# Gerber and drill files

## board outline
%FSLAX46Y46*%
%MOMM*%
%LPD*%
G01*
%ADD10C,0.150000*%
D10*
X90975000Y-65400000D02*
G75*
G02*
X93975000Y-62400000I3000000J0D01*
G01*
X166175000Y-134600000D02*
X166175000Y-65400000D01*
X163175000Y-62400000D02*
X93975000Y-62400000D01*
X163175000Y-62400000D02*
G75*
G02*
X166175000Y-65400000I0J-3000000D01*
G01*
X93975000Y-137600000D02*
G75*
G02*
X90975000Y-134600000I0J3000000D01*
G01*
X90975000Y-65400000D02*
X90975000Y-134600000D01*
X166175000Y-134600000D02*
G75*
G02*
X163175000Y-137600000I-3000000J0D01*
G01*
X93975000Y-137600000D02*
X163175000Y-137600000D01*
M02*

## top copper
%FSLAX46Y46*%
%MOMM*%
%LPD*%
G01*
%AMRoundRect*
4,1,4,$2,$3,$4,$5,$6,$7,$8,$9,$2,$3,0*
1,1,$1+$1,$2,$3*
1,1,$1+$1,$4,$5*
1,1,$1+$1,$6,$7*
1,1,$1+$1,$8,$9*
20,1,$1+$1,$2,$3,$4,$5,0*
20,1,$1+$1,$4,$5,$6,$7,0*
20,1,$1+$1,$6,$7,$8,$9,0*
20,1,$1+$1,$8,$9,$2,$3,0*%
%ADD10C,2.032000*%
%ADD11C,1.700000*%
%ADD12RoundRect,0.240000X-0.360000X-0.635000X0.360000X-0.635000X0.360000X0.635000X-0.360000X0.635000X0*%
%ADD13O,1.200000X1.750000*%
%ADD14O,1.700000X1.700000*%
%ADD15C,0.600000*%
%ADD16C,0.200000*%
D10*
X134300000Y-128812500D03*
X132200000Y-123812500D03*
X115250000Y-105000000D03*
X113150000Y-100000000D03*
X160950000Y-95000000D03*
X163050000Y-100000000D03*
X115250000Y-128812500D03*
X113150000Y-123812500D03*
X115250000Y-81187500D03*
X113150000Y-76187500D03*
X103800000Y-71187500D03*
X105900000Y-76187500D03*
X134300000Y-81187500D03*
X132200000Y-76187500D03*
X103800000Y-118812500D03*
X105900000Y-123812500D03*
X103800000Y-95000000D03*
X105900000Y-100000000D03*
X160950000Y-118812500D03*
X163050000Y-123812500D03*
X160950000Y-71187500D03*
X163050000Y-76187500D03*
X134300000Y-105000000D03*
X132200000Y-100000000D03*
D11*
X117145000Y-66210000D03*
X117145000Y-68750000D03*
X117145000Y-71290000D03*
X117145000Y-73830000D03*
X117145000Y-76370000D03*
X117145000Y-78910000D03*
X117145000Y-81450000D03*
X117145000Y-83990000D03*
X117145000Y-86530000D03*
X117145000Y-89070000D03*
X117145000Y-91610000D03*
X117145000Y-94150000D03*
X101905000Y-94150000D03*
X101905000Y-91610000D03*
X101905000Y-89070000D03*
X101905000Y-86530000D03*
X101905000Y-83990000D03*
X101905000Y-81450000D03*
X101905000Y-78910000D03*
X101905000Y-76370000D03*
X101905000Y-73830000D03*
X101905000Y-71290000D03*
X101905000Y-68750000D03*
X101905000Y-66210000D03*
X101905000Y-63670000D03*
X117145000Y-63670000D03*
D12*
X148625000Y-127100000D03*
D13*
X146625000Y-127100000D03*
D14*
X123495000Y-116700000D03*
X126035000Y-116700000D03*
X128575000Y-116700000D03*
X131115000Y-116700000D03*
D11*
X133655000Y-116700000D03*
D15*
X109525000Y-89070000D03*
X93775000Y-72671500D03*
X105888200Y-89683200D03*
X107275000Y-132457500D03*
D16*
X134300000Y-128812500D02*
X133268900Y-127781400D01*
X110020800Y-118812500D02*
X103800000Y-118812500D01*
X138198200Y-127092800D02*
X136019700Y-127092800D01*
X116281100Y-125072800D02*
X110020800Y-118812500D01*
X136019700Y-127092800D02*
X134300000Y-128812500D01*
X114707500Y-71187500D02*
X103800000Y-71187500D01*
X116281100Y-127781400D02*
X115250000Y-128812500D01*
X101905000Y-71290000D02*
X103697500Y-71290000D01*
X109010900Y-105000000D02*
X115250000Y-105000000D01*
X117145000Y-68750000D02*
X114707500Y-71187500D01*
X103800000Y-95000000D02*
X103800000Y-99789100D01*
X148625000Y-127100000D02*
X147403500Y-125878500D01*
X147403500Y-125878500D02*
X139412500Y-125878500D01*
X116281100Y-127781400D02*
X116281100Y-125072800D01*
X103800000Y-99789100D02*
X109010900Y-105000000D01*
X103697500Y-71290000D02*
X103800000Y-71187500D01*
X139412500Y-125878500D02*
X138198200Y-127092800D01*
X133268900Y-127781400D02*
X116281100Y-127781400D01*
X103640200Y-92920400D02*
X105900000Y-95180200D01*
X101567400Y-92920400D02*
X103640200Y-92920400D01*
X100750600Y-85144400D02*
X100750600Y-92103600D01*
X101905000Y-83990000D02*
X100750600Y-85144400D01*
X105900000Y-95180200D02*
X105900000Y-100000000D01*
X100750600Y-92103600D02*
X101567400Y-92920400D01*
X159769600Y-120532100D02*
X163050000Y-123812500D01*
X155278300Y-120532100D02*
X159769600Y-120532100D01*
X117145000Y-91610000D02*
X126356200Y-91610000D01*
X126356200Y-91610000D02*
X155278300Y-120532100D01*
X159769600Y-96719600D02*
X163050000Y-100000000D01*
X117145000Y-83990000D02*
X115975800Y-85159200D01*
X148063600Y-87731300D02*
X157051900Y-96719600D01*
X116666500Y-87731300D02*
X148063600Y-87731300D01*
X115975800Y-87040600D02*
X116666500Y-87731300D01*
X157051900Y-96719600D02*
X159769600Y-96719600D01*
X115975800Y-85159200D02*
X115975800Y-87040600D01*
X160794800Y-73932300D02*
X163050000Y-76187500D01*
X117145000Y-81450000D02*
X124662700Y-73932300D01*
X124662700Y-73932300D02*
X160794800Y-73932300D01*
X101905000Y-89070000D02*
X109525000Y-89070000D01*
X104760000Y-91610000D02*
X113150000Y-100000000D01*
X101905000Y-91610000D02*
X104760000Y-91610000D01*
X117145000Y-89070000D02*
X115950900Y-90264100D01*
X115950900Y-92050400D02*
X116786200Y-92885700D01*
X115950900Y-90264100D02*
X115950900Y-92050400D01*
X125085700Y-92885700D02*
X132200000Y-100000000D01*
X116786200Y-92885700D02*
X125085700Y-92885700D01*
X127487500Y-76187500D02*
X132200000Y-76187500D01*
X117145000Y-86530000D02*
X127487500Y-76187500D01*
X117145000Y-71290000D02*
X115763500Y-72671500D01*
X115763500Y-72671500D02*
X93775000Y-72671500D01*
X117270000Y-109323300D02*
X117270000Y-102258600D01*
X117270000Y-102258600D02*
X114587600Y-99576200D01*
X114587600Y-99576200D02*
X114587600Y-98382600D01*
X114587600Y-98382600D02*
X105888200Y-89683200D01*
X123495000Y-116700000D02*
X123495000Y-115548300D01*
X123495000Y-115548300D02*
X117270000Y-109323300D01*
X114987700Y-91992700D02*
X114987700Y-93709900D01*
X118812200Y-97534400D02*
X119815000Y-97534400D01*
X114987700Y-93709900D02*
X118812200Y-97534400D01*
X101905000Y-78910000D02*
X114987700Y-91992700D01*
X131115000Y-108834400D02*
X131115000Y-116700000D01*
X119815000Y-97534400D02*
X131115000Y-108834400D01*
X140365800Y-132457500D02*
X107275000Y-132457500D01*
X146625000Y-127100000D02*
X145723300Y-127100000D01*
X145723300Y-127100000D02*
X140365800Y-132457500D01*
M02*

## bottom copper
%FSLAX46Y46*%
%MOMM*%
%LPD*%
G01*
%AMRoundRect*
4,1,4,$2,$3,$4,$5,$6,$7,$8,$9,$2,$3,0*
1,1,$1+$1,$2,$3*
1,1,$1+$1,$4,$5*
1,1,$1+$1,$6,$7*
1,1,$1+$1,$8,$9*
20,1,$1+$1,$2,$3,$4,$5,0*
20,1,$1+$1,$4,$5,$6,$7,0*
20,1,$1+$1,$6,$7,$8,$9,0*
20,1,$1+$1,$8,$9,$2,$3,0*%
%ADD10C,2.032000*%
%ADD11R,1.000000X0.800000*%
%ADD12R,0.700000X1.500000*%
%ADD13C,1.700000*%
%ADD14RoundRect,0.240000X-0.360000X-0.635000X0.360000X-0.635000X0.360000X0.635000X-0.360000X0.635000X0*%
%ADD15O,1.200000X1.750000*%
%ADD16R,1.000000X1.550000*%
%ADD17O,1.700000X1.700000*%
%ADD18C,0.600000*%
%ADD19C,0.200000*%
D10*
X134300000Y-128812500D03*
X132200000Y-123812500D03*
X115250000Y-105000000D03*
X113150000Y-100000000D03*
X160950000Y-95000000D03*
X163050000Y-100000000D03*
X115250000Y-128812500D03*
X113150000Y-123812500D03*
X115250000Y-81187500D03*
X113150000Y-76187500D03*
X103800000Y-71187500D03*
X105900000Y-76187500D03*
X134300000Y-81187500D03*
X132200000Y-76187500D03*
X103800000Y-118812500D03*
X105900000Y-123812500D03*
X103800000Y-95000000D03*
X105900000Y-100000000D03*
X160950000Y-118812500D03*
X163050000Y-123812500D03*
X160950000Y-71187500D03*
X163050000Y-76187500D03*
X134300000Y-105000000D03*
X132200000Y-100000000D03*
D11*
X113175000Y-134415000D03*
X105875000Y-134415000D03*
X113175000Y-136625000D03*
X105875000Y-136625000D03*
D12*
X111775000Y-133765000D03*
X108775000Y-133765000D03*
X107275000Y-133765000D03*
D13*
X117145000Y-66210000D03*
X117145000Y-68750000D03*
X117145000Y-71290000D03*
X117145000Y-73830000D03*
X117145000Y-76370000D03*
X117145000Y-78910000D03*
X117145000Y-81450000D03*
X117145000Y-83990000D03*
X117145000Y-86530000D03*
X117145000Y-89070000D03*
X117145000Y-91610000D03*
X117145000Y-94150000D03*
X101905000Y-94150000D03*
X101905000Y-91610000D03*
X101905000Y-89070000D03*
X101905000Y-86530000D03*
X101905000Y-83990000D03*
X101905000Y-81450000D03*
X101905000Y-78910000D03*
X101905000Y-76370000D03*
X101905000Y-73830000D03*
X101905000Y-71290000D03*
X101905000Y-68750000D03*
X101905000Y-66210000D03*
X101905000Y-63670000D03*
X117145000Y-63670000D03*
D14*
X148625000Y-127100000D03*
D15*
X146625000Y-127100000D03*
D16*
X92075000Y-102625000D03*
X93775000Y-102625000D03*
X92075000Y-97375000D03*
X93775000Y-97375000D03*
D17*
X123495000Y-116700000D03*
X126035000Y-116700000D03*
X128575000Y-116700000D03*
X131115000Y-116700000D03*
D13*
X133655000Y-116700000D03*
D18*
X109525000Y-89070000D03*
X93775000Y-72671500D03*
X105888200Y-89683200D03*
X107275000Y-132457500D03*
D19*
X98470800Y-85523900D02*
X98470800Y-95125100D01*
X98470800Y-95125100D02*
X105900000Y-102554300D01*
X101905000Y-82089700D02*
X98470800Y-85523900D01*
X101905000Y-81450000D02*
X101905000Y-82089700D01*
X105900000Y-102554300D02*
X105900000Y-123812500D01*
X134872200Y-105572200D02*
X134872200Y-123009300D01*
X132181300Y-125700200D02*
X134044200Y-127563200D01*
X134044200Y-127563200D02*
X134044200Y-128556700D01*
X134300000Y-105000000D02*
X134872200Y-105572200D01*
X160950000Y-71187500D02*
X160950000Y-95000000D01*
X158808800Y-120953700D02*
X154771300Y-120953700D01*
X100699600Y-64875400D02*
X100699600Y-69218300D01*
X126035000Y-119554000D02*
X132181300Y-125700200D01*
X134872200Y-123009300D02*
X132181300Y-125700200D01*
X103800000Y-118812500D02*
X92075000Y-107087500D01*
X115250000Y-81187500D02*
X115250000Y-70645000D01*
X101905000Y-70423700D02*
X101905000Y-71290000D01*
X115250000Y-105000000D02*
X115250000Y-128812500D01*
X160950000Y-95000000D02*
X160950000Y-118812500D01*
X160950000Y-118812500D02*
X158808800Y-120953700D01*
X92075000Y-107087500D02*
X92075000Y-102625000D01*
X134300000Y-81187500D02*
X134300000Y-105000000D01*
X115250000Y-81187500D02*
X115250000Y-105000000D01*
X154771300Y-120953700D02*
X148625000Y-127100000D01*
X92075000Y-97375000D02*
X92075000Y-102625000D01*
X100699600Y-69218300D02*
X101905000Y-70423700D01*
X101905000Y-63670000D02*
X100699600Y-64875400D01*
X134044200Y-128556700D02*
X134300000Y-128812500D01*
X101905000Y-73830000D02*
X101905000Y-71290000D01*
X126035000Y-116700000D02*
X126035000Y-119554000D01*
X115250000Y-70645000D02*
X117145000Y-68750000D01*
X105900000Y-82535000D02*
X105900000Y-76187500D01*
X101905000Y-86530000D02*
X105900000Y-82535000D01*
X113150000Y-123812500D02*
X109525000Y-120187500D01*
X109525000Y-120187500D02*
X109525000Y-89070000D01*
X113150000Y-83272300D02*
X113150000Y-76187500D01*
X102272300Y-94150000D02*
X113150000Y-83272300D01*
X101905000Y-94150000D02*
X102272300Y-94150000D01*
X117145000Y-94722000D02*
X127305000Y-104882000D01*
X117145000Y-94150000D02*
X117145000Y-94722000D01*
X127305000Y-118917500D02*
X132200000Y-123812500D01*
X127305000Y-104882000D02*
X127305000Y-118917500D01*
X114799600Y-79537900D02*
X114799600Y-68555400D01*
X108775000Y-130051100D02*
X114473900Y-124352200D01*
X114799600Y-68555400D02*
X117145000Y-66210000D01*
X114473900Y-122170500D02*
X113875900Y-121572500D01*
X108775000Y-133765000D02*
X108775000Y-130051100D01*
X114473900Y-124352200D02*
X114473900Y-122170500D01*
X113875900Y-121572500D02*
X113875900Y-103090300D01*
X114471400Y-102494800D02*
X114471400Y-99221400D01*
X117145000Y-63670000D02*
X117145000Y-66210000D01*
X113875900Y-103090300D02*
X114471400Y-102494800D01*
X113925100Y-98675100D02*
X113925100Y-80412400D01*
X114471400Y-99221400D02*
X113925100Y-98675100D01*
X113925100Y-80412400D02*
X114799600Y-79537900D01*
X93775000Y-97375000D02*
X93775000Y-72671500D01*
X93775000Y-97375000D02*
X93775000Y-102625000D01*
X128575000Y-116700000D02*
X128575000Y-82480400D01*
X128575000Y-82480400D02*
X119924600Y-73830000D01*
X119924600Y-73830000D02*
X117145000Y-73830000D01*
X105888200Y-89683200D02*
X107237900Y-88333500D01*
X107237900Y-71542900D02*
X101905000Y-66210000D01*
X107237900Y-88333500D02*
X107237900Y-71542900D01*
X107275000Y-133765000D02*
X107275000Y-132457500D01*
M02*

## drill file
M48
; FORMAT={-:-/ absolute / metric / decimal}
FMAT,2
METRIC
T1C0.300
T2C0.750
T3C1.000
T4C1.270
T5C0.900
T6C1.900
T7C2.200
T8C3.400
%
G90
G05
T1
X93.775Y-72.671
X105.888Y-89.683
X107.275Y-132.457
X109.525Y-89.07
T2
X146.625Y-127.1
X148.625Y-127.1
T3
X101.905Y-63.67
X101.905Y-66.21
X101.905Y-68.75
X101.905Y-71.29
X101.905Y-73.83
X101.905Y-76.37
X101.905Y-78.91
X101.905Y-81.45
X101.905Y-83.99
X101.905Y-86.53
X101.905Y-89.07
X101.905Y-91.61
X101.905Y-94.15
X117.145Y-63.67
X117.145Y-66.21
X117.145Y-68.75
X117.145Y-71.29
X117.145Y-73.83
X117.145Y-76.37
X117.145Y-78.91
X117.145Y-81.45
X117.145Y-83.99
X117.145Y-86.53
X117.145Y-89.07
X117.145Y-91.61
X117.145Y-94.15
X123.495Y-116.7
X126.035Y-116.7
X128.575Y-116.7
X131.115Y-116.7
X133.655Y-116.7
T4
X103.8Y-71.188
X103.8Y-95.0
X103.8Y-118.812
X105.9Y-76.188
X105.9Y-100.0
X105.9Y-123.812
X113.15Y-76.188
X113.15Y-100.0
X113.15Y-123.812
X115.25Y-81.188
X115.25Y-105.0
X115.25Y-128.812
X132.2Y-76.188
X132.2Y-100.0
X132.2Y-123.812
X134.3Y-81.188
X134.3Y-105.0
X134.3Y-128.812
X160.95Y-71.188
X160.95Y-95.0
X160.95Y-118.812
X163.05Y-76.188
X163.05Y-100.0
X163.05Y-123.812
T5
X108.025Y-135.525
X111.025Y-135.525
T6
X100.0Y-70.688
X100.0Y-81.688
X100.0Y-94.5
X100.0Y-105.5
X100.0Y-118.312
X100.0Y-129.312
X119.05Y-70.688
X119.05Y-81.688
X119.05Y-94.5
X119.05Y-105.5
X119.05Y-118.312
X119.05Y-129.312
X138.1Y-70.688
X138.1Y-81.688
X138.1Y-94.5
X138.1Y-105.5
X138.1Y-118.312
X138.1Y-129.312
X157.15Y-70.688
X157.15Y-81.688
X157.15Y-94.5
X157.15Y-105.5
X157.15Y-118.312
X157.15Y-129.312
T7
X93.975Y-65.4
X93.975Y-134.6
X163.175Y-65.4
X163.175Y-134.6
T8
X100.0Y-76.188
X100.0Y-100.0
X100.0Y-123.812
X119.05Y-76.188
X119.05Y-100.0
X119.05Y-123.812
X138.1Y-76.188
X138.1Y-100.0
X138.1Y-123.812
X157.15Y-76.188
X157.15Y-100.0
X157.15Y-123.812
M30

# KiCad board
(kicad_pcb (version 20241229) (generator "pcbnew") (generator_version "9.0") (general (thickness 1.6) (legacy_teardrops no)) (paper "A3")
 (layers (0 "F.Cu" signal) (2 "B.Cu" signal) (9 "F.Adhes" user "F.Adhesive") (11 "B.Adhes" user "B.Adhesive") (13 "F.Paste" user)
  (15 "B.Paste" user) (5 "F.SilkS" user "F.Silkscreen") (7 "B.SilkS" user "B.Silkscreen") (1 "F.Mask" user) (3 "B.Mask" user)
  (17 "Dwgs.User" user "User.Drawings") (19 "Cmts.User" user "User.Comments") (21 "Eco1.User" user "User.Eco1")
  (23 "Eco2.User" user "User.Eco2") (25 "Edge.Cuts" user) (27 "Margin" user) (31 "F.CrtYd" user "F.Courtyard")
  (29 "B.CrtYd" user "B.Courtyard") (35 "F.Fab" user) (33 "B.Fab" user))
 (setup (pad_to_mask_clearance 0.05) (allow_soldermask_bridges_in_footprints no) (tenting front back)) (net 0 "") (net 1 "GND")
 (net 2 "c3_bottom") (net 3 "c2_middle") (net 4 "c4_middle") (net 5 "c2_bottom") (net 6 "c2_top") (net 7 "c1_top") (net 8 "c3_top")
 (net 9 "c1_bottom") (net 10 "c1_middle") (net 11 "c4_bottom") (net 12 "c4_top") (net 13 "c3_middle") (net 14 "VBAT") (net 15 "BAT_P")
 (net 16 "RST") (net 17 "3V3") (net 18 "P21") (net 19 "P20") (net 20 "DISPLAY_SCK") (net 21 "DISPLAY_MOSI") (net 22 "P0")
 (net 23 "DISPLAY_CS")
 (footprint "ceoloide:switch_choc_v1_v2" (layer "F.Cu") (at 138.1 123.8125 90)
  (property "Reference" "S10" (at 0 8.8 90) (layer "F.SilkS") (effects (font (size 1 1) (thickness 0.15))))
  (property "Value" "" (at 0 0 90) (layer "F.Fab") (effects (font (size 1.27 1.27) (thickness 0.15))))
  (pad "" np_thru_hole circle (at -5.5 0 90) (size 1.9 1.9) (drill 1.9) (layers "*.Cu" "*.Mask"))
  (pad "" np_thru_hole circle (at 0 0 90) (size 3.4 3.4) (drill 3.4) (layers "*.Cu" "*.Mask"))
  (pad "" np_thru_hole circle (at 5.5 0 90) (size 1.9 1.9) (drill 1.9) (layers "*.Cu" "*.Mask"))
  (pad "1" thru_hole circle (at -5 -3.8 285) (size 2.032 2.032) (drill 1.27) (layers "*.Cu" "*.Mask") (remove_unused_layers no)
   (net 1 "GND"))
  (pad "2" thru_hole circle (at 0 -5.9 285) (size 2.032 2.032) (drill 1.27) (layers "*.Cu" "*.Mask") (remove_unused_layers no)
   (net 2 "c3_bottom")))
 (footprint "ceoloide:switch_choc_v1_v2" (layer "F.Cu") (at 119.05 100 90)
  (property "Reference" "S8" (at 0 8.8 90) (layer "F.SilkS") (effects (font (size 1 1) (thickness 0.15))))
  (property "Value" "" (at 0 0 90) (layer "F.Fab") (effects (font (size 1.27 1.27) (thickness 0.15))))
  (pad "" np_thru_hole circle (at -5.5 0 90) (size 1.9 1.9) (drill 1.9) (layers "*.Cu" "*.Mask"))
  (pad "" np_thru_hole circle (at 0 0 90) (size 3.4 3.4) (drill 3.4) (layers "*.Cu" "*.Mask"))
  (pad "" np_thru_hole circle (at 5.5 0 90) (size 1.9 1.9) (drill 1.9) (layers "*.Cu" "*.Mask"))
  (pad "1" thru_hole circle (at -5 -3.8 285) (size 2.032 2.032) (drill 1.27) (layers "*.Cu" "*.Mask") (remove_unused_layers no)
   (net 1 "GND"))
  (pad "2" thru_hole circle (at 0 -5.9 285) (size 2.032 2.032) (drill 1.27) (layers "*.Cu" "*.Mask") (remove_unused_layers no)
   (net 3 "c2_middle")))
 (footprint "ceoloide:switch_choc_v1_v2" (layer "F.Cu") (at 157.15 100 -90)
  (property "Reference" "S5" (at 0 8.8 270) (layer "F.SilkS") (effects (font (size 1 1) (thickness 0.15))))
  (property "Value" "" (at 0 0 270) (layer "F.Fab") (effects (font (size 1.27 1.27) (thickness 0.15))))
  (pad "" np_thru_hole circle (at -5.5 0 270) (size 1.9 1.9) (drill 1.9) (layers "*.Cu" "*.Mask"))
  (pad "" np_thru_hole circle (at 0 0 270) (size 3.4 3.4) (drill 3.4) (layers "*.Cu" "*.Mask"))
  (pad "" np_thru_hole circle (at 5.5 0 270) (size 1.9 1.9) (drill 1.9) (layers "*.Cu" "*.Mask"))
  (pad "1" thru_hole circle (at -5 -3.8 105) (size 2.032 2.032) (drill 1.27) (layers "*.Cu" "*.Mask") (remove_unused_layers no)
   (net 1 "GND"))
  (pad "2" thru_hole circle (at 0 -5.9 105) (size 2.032 2.032) (drill 1.27) (layers "*.Cu" "*.Mask") (remove_unused_layers no)
   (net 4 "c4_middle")))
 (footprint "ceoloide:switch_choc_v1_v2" (layer "F.Cu") (at 119.05 123.8125 90)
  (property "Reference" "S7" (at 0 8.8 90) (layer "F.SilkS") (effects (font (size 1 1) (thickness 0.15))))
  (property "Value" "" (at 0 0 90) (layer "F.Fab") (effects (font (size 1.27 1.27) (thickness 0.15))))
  (pad "" np_thru_hole circle (at -5.5 0 90) (size 1.9 1.9) (drill 1.9) (layers "*.Cu" "*.Mask"))
  (pad "" np_thru_hole circle (at 0 0 90) (size 3.4 3.4) (drill 3.4) (layers "*.Cu" "*.Mask"))
  (pad "" np_thru_hole circle (at 5.5 0 90) (size 1.9 1.9) (drill 1.9) (layers "*.Cu" "*.Mask"))
  (pad "1" thru_hole circle (at -5 -3.8 285) (size 2.032 2.032) (drill 1.27) (layers "*.Cu" "*.Mask") (remove_unused_layers no)
   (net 1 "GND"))
  (pad "2" thru_hole circle (at 0 -5.9 285) (size 2.032 2.032) (drill 1.27) (layers "*.Cu" "*.Mask") (remove_unused_layers no)
   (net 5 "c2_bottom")))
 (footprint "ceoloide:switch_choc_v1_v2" (layer "F.Cu") (at 119.05 76.1875 90)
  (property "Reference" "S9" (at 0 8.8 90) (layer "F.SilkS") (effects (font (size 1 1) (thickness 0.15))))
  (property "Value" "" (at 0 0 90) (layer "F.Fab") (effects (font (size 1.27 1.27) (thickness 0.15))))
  (pad "" np_thru_hole circle (at -5.5 0 90) (size 1.9 1.9) (drill 1.9) (layers "*.Cu" "*.Mask"))
  (pad "" np_thru_hole circle (at 0 0 90) (size 3.4 3.4) (drill 3.4) (layers "*.Cu" "*.Mask"))
  (pad "" np_thru_hole circle (at 5.5 0 90) (size 1.9 1.9) (drill 1.9) (layers "*.Cu" "*.Mask"))
  (pad "1" thru_hole circle (at -5 -3.8 285) (size 2.032 2.032) (drill 1.27) (layers "*.Cu" "*.Mask") (remove_unused_layers no)
   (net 1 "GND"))
  (pad "2" thru_hole circle (at 0 -5.9 285) (size 2.032 2.032) (drill 1.27) (layers "*.Cu" "*.Mask") (remove_unused_layers no)
   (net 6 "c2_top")))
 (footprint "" (layer "F.Cu") (at 128.574999 100)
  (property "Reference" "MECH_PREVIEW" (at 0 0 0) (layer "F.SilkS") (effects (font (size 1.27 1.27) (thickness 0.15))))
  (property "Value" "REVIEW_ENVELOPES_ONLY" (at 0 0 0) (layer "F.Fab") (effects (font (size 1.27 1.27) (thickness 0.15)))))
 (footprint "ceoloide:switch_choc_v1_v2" (layer "F.Cu") (at 100 76.1875 -90)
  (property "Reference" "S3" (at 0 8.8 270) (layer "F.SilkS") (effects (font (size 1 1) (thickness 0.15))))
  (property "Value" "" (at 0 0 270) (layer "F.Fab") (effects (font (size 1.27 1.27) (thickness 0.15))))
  (pad "" np_thru_hole circle (at -5.5 0 270) (size 1.9 1.9) (drill 1.9) (layers "*.Cu" "*.Mask"))
  (pad "" np_thru_hole circle (at 0 0 270) (size 3.4 3.4) (drill 3.4) (layers "*.Cu" "*.Mask"))
  (pad "" np_thru_hole circle (at 5.5 0 270) (size 1.9 1.9) (drill 1.9) (layers "*.Cu" "*.Mask"))
  (pad "1" thru_hole circle (at -5 -3.8 105) (size 2.032 2.032) (drill 1.27) (layers "*.Cu" "*.Mask") (remove_unused_layers no)
   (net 1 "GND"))
  (pad "2" thru_hole circle (at 0 -5.9 105) (size 2.032 2.032) (drill 1.27) (layers "*.Cu" "*.Mask") (remove_unused_layers no)
   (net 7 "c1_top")))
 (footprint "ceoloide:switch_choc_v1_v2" (layer "F.Cu") (at 138.1 76.1875 90)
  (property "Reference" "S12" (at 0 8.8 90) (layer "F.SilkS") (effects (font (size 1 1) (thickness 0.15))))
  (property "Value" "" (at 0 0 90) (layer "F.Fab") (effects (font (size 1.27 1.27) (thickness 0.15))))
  (pad "" np_thru_hole circle (at -5.5 0 90) (size 1.9 1.9) (drill 1.9) (layers "*.Cu" "*.Mask"))
  (pad "" np_thru_hole circle (at 0 0 90) (size 3.4 3.4) (drill 3.4) (layers "*.Cu" "*.Mask"))
  (pad "" np_thru_hole circle (at 5.5 0 90) (size 1.9 1.9) (drill 1.9) (layers "*.Cu" "*.Mask"))
  (pad "1" thru_hole circle (at -5 -3.8 285) (size 2.032 2.032) (drill 1.27) (layers "*.Cu" "*.Mask") (remove_unused_layers no)
   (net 1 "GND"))
  (pad "2" thru_hole circle (at 0 -5.9 285) (size 2.032 2.032) (drill 1.27) (layers "*.Cu" "*.Mask") (remove_unused_layers no)
   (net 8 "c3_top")))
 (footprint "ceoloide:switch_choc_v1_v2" (layer "F.Cu") (at 100 123.8125 -90)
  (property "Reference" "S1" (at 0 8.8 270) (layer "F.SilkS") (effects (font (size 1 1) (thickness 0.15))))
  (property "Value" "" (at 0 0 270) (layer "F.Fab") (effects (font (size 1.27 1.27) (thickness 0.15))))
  (pad "" np_thru_hole circle (at -5.5 0 270) (size 1.9 1.9) (drill 1.9) (layers "*.Cu" "*.Mask"))
  (pad "" np_thru_hole circle (at 0 0 270) (size 3.4 3.4) (drill 3.4) (layers "*.Cu" "*.Mask"))
  (pad "" np_thru_hole circle (at 5.5 0 270) (size 1.9 1.9) (drill 1.9) (layers "*.Cu" "*.Mask"))
  (pad "1" thru_hole circle (at -5 -3.8 105) (size 2.032 2.032) (drill 1.27) (layers "*.Cu" "*.Mask") (remove_unused_layers no)
   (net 1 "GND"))
  (pad "2" thru_hole circle (at 0 -5.9 105) (size 2.032 2.032) (drill 1.27) (layers "*.Cu" "*.Mask") (remove_unused_layers no)
   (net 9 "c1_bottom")))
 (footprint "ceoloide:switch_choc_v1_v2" (layer "F.Cu") (at 100 100 -90)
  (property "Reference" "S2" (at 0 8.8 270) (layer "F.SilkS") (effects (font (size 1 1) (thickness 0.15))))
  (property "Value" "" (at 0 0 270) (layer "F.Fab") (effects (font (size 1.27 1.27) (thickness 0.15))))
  (pad "" np_thru_hole circle (at -5.5 0 270) (size 1.9 1.9) (drill 1.9) (layers "*.Cu" "*.Mask"))
  (pad "" np_thru_hole circle (at 0 0 270) (size 3.4 3.4) (drill 3.4) (layers "*.Cu" "*.Mask"))
  (pad "" np_thru_hole circle (at 5.5 0 270) (size 1.9 1.9) (drill 1.9) (layers "*.Cu" "*.Mask"))
  (pad "1" thru_hole circle (at -5 -3.8 105) (size 2.032 2.032) (drill 1.27) (layers "*.Cu" "*.Mask") (remove_unused_layers no)
   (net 1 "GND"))
  (pad "2" thru_hole circle (at 0 -5.9 105) (size 2.032 2.032) (drill 1.27) (layers "*.Cu" "*.Mask") (remove_unused_layers no)
   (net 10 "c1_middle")))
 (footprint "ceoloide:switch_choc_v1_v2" (layer "F.Cu") (at 157.15 123.8125 -90)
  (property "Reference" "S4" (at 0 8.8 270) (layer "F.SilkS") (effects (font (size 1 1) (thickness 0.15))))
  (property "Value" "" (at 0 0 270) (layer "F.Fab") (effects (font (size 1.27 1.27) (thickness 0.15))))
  (pad "" np_thru_hole circle (at -5.5 0 270) (size 1.9 1.9) (drill 1.9) (layers "*.Cu" "*.Mask"))
  (pad "" np_thru_hole circle (at 0 0 270) (size 3.4 3.4) (drill 3.4) (layers "*.Cu" "*.Mask"))
  (pad "" np_thru_hole circle (at 5.5 0 270) (size 1.9 1.9) (drill 1.9) (layers "*.Cu" "*.Mask"))
  (pad "1" thru_hole circle (at -5 -3.8 105) (size 2.032 2.032) (drill 1.27) (layers "*.Cu" "*.Mask") (remove_unused_layers no)
   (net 1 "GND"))
  (pad "2" thru_hole circle (at 0 -5.9 105) (size 2.032 2.032) (drill 1.27) (layers "*.Cu" "*.Mask") (remove_unused_layers no)
   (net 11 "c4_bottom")))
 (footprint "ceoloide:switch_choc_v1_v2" (layer "F.Cu") (at 157.15 76.1875 -90)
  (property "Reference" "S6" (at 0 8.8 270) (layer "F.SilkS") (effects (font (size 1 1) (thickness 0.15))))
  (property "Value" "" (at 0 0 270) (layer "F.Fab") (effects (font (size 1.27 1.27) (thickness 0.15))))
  (pad "" np_thru_hole circle (at -5.5 0 270) (size 1.9 1.9) (drill 1.9) (layers "*.Cu" "*.Mask"))
  (pad "" np_thru_hole circle (at 0 0 270) (size 3.4 3.4) (drill 3.4) (layers "*.Cu" "*.Mask"))
  (pad "" np_thru_hole circle (at 5.5 0 270) (size 1.9 1.9) (drill 1.9) (layers "*.Cu" "*.Mask"))
  (pad "1" thru_hole circle (at -5 -3.8 105) (size 2.032 2.032) (drill 1.27) (layers "*.Cu" "*.Mask") (remove_unused_layers no)
   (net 1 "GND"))
  (pad "2" thru_hole circle (at 0 -5.9 105) (size 2.032 2.032) (drill 1.27) (layers "*.Cu" "*.Mask") (remove_unused_layers no)
   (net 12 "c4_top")))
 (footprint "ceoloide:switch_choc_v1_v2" (layer "F.Cu") (at 138.1 100 90)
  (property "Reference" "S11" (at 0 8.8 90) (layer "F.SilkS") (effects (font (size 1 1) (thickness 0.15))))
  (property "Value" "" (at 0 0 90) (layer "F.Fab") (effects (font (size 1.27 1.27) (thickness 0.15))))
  (pad "" np_thru_hole circle (at -5.5 0 90) (size 1.9 1.9) (drill 1.9) (layers "*.Cu" "*.Mask"))
  (pad "" np_thru_hole circle (at 0 0 90) (size 3.4 3.4) (drill 3.4) (layers "*.Cu" "*.Mask"))
  (pad "" np_thru_hole circle (at 5.5 0 90) (size 1.9 1.9) (drill 1.9) (layers "*.Cu" "*.Mask"))
  (pad "1" thru_hole circle (at -5 -3.8 285) (size 2.032 2.032) (drill 1.27) (layers "*.Cu" "*.Mask") (remove_unused_layers no)
   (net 1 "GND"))
  (pad "2" thru_hole circle (at 0 -5.9 285) (size 2.032 2.032) (drill 1.27) (layers "*.Cu" "*.Mask") (remove_unused_layers no)
   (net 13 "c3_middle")))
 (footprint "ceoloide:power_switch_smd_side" (layer "B.Cu") (at 109.525 135.5 -90)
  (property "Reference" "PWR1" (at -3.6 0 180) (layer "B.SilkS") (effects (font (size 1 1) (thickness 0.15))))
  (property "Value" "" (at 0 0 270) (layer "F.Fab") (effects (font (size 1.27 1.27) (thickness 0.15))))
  (pad "" smd rect (at -1.085 -3.65 180) (size 1 0.8) (layers "B.Cu" "B.Mask" "B.Paste"))
  (pad "" smd rect (at -1.085 3.65 180) (size 1 0.8) (layers "B.Cu" "B.Mask" "B.Paste"))
  (pad "" np_thru_hole circle (at 0.025 -1.5) (size 0.9 0.9) (drill 0.9) (layers "*.Cu" "*.Mask"))
  (pad "" np_thru_hole circle (at 0.025 1.5) (size 0.9 0.9) (drill 0.9) (layers "*.Cu" "*.Mask"))
  (pad "" smd rect (at 1.125 -3.65 180) (size 1 0.8) (layers "B.Cu" "B.Mask" "B.Paste"))
  (pad "" smd rect (at 1.125 3.65 180) (size 1 0.8) (layers "B.Cu" "B.Mask" "B.Paste"))
  (pad "1" smd rect (at -1.735 -2.25 180) (size 0.7 1.5) (layers "B.Cu" "B.Mask" "B.Paste"))
  (pad "2" smd rect (at -1.735 0.75 180) (size 0.7 1.5) (layers "B.Cu" "B.Mask" "B.Paste") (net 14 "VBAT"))
  (pad "3" smd rect (at -1.735 2.25 180) (size 0.7 1.5) (layers "B.Cu" "B.Mask" "B.Paste") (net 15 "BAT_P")))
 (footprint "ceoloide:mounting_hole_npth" (layer "B.Cu") (at 93.975 134.6)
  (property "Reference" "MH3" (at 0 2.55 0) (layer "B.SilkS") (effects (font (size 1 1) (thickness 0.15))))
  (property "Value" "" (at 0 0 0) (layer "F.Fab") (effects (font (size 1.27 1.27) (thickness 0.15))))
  (pad "" np_thru_hole circle (at 0 0) (size 2.2 2.2) (drill 2.2) (layers "*.Cu" "*.Mask")))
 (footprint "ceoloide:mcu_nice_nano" (layer "B.Cu") (at 109.525 78.91)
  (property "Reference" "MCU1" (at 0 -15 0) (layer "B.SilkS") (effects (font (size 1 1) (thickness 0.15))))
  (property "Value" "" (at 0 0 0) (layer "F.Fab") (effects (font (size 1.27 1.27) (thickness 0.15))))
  (pad "1" thru_hole circle (at 7.62 -12.7) (size 1.7 1.7) (drill 1) (layers "*.Cu" "*.Mask") (remove_unused_layers no) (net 14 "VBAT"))
  (pad "2" thru_hole circle (at 7.62 -10.16) (size 1.7 1.7) (drill 1) (layers "*.Cu" "*.Mask") (remove_unused_layers no) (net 1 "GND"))
  (pad "3" thru_hole circle (at 7.62 -7.62) (size 1.7 1.7) (drill 1) (layers "*.Cu" "*.Mask") (remove_unused_layers no) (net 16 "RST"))
  (pad "4" thru_hole circle (at 7.62 -5.08) (size 1.7 1.7) (drill 1) (layers "*.Cu" "*.Mask") (remove_unused_layers no) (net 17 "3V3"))
  (pad "5" thru_hole circle (at 7.62 -2.54) (size 1.7 1.7) (drill 1) (layers "*.Cu" "*.Mask") (remove_unused_layers no) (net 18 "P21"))
  (pad "6" thru_hole circle (at 7.62 0) (size 1.7 1.7) (drill 1) (layers "*.Cu" "*.Mask") (remove_unused_layers no) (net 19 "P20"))
  (pad "7" thru_hole circle (at 7.62 2.54) (size 1.7 1.7) (drill 1) (layers "*.Cu" "*.Mask") (remove_unused_layers no) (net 12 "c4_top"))
  (pad "8" thru_hole circle (at 7.62 5.08) (size 1.7 1.7) (drill 1) (layers "*.Cu" "*.Mask") (remove_unused_layers no) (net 4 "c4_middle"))
  (pad "9" thru_hole circle (at 7.62 7.62) (size 1.7 1.7) (drill 1) (layers "*.Cu" "*.Mask") (remove_unused_layers no) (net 8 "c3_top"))
  (pad "10" thru_hole circle (at 7.62 10.16) (size 1.7 1.7) (drill 1) (layers "*.Cu" "*.Mask") (remove_unused_layers no)
   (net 13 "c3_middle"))
  (pad "11" thru_hole circle (at 7.62 12.7) (size 1.7 1.7) (drill 1) (layers "*.Cu" "*.Mask") (remove_unused_layers no) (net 11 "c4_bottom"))
  (pad "12" thru_hole circle (at 7.62 15.24) (size 1.7 1.7) (drill 1) (layers "*.Cu" "*.Mask") (remove_unused_layers no) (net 2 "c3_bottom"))
  (pad "13" thru_hole circle (at -7.62 15.24) (size 1.7 1.7) (drill 1) (layers "*.Cu" "*.Mask") (remove_unused_layers no) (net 6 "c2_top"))
  (pad "14" thru_hole circle (at -7.62 12.7) (size 1.7 1.7) (drill 1) (layers "*.Cu" "*.Mask") (remove_unused_layers no) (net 3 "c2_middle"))
  (pad "15" thru_hole circle (at -7.62 10.16) (size 1.7 1.7) (drill 1) (layers "*.Cu" "*.Mask") (remove_unused_layers no)
   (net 5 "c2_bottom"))
  (pad "16" thru_hole circle (at -7.62 7.62) (size 1.7 1.7) (drill 1) (layers "*.Cu" "*.Mask") (remove_unused_layers no) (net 7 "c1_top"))
  (pad "17" thru_hole circle (at -7.62 5.08) (size 1.7 1.7) (drill 1) (layers "*.Cu" "*.Mask") (remove_unused_layers no)
   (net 10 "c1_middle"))
  (pad "18" thru_hole circle (at -7.62 2.54) (size 1.7 1.7) (drill 1) (layers "*.Cu" "*.Mask") (remove_unused_layers no) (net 9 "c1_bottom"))
  (pad "19" thru_hole circle (at -7.62 0) (size 1.7 1.7) (drill 1) (layers "*.Cu" "*.Mask") (remove_unused_layers no) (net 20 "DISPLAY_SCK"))
  (pad "20" thru_hole circle (at -7.62 -2.54) (size 1.7 1.7) (drill 1) (layers "*.Cu" "*.Mask") (remove_unused_layers no)
   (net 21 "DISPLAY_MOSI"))
  (pad "21" thru_hole circle (at -7.62 -5.08) (size 1.7 1.7) (drill 1) (layers "*.Cu" "*.Mask") (remove_unused_layers no) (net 1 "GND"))
  (pad "22" thru_hole circle (at -7.62 -7.62) (size 1.7 1.7) (drill 1) (layers "*.Cu" "*.Mask") (remove_unused_layers no) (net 1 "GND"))
  (pad "23" thru_hole circle (at -7.62 -10.16) (size 1.7 1.7) (drill 1) (layers "*.Cu" "*.Mask") (remove_unused_layers no) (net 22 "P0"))
  (pad "24" thru_hole circle (at -7.62 -12.7) (size 1.7 1.7) (drill 1) (layers "*.Cu" "*.Mask") (remove_unused_layers no)
   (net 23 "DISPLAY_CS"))
  (pad "25" thru_hole circle (at -7.62 -15.24) (size 1.7 1.7) (drill 1) (layers "*.Cu" "*.Mask") (remove_unused_layers no) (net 1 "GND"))
  (pad "26" thru_hole circle (at 7.62 -15.24) (size 1.7 1.7) (drill 1) (layers "*.Cu" "*.Mask") (remove_unused_layers no) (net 14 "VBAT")))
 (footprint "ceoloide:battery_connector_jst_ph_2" (layer "B.Cu") (at 147.625 127.1)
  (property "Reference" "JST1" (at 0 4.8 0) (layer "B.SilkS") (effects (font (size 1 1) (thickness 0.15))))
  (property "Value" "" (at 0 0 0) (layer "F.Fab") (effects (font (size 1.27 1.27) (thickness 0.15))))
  (pad "1" thru_hole roundrect (at 1 0) (size 1.2 1.75) (drill 0.75) (layers "*.Cu" "*.Mask") (remove_unused_layers no)
   (roundrect_rratio 0.2) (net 1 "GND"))
  (pad "2" thru_hole oval (at -1 0) (size 1.2 1.75) (drill 0.75) (layers "*.Cu" "*.Mask") (remove_unused_layers no) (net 15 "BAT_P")))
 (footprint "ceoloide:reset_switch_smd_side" (layer "B.Cu") (at 92.925 100 90)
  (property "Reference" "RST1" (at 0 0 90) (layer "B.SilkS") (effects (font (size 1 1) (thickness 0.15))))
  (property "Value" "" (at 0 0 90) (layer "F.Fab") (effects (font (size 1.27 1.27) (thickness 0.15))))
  (pad "1" smd rect (at -2.625 -0.85 270) (size 1.55 1) (layers "B.Cu" "B.Mask" "B.Paste") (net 1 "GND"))
  (pad "2" smd rect (at -2.625 0.85 270) (size 1.55 1) (layers "B.Cu" "B.Mask" "B.Paste") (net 16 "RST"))
  (pad "3" smd rect (at 2.625 -0.85 270) (size 1.55 1) (layers "B.Cu" "B.Mask" "B.Paste") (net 1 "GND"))
  (pad "4" smd rect (at 2.625 0.85 270) (size 1.55 1) (layers "B.Cu" "B.Mask" "B.Paste") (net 16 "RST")))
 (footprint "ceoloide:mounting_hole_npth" (layer "B.Cu") (at 163.175 65.4)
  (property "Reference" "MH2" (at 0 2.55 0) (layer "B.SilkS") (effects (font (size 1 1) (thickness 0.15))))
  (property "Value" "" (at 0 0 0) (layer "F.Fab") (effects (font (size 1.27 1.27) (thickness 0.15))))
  (pad "" np_thru_hole circle (at 0 0) (size 2.2 2.2) (drill 2.2) (layers "*.Cu" "*.Mask")))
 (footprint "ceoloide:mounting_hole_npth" (layer "B.Cu") (at 163.175 134.6)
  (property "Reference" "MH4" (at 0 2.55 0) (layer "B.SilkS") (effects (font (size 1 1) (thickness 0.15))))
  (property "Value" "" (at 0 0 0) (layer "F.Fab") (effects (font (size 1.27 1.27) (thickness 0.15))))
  (pad "" np_thru_hole circle (at 0 0) (size 2.2 2.2) (drill 2.2) (layers "*.Cu" "*.Mask")))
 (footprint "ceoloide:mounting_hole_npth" (layer "B.Cu") (at 93.975 65.4)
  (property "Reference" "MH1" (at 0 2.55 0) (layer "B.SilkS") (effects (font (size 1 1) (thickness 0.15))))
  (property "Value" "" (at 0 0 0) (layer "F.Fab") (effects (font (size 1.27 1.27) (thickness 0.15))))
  (pad "" np_thru_hole circle (at 0 0) (size 2.2 2.2) (drill 2.2) (layers "*.Cu" "*.Mask")))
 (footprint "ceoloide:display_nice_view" (layer "B.Cu") (at 128.575 100)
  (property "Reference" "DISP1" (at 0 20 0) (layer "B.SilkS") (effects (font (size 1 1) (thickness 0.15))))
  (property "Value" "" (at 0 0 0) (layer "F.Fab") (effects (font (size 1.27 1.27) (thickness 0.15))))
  (pad "1" thru_hole oval (at -5.08 16.7 270) (size 1.7 1.7) (drill 1) (layers "*.Cu" "*.Mask") (remove_unused_layers no)
   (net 23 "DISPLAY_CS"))
  (pad "2" thru_hole oval (at -2.54 16.7 270) (size 1.7 1.7) (drill 1) (layers "*.Cu" "*.Mask") (remove_unused_layers no) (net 1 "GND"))
  (pad "3" thru_hole oval (at 0 16.7 270) (size 1.7 1.7) (drill 1) (layers "*.Cu" "*.Mask") (remove_unused_layers no) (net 17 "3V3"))
  (pad "4" thru_hole oval (at 2.54 16.7 270) (size 1.7 1.7) (drill 1) (layers "*.Cu" "*.Mask") (remove_unused_layers no)
   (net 20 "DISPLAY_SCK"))
  (pad "5" thru_hole circle (at 5.08 16.7 270) (size 1.7 1.7) (drill 1) (layers "*.Cu" "*.Mask") (remove_unused_layers no)
   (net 21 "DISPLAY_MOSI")))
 (gr_arc (start 90.975 65.4) (mid 91.85368 63.27868) (end 93.975 62.4) (stroke (width 0.15) (type default)) (layer "Edge.Cuts"))
 (gr_line (start 166.175 134.6) (end 166.175 65.4) (stroke (width 0.15) (type default)) (layer "Edge.Cuts"))
 (gr_line (start 163.175 62.4) (end 93.975 62.4) (stroke (width 0.15) (type default)) (layer "Edge.Cuts"))
 (gr_arc (start 163.175 62.4) (mid 165.29632 63.27868) (end 166.175 65.4) (stroke (width 0.15) (type default)) (layer "Edge.Cuts"))
 (gr_arc (start 93.975 137.6) (mid 91.85368 136.72132) (end 90.975 134.6) (stroke (width 0.15) (type default)) (layer "Edge.Cuts"))
 (gr_line (start 90.975 65.4) (end 90.975 134.6) (stroke (width 0.15) (type default)) (layer "Edge.Cuts"))
 (gr_arc (start 166.175 134.6) (mid 165.29632 136.72132) (end 163.175 137.6) (stroke (width 0.15) (type default)) (layer "Edge.Cuts"))
 (gr_line (start 93.975 137.6) (end 163.175 137.6) (stroke (width 0.15) (type default)) (layer "Edge.Cuts"))
 (segment (start 98.4708 85.5239) (end 98.4708 95.1251) (width 0.2) (layer "B.Cu") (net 9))
 (segment (start 98.4708 95.1251) (end 105.9 102.5543) (width 0.2) (layer "B.Cu") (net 9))
 (segment (start 101.905 82.0897) (end 98.4708 85.5239) (width 0.2) (layer "B.Cu") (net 9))
 (segment (start 101.905 81.45) (end 101.905 82.0897) (width 0.2) (layer "B.Cu") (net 9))
 (segment (start 105.9 102.5543) (end 105.9 123.8125) (width 0.2) (layer "B.Cu") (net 9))
 (segment (start 134.3 128.8125) (end 133.2689 127.7814) (width 0.2) (layer "F.Cu") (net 1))
 (segment (start 110.0208 118.8125) (end 103.8 118.8125) (width 0.2) (layer "F.Cu") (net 1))
 (segment (start 138.1982 127.0928) (end 136.0197 127.0928) (width 0.2) (layer "F.Cu") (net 1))
 (segment (start 116.2811 125.0728) (end 110.0208 118.8125) (width 0.2) (layer "F.Cu") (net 1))
 (segment (start 136.0197 127.0928) (end 134.3 128.8125) (width 0.2) (layer "F.Cu") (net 1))
 (segment (start 114.7075 71.1875) (end 103.8 71.1875) (width 0.2) (layer "F.Cu") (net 1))
 (segment (start 116.2811 127.7814) (end 115.25 128.8125) (width 0.2) (layer "F.Cu") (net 1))
 (segment (start 101.905 71.29) (end 103.6975 71.29) (width 0.2) (layer "F.Cu") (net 1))
 (segment (start 109.0109 105) (end 115.25 105) (width 0.2) (layer "F.Cu") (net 1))
 (segment (start 117.145 68.75) (end 114.7075 71.1875) (width 0.2) (layer "F.Cu") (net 1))
 (segment (start 103.8 95) (end 103.8 99.7891) (width 0.2) (layer "F.Cu") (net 1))
 (segment (start 148.625 127.1) (end 147.4035 125.8785) (width 0.2) (layer "F.Cu") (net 1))
 (segment (start 147.4035 125.8785) (end 139.4125 125.8785) (width 0.2) (layer "F.Cu") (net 1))
 (segment (start 116.2811 127.7814) (end 116.2811 125.0728) (width 0.2) (layer "F.Cu") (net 1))
 (segment (start 103.8 99.7891) (end 109.0109 105) (width 0.2) (layer "F.Cu") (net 1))
 (segment (start 103.6975 71.29) (end 103.8 71.1875) (width 0.2) (layer "F.Cu") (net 1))
 (segment (start 139.4125 125.8785) (end 138.1982 127.0928) (width 0.2) (layer "F.Cu") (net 1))
 (segment (start 133.2689 127.7814) (end 116.2811 127.7814) (width 0.2) (layer "F.Cu") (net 1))
 (segment (start 134.8722 105.5722) (end 134.8722 123.0093) (width 0.2) (layer "B.Cu") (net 1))
 (segment (start 132.1813 125.7002) (end 134.0442 127.5632) (width 0.2) (layer "B.Cu") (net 1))
 (segment (start 134.0442 127.5632) (end 134.0442 128.5567) (width 0.2) (layer "B.Cu") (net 1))
 (segment (start 134.3 105) (end 134.8722 105.5722) (width 0.2) (layer "B.Cu") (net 1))
 (segment (start 160.95 71.1875) (end 160.95 95) (width 0.2) (layer "B.Cu") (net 1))
 (segment (start 158.8088 120.9537) (end 154.7713 120.9537) (width 0.2) (layer "B.Cu") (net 1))
 (segment (start 100.6996 64.8754) (end 100.6996 69.2183) (width 0.2) (layer "B.Cu") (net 1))
 (segment (start 126.035 119.554) (end 132.1813 125.7002) (width 0.2) (layer "B.Cu") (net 1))
 (segment (start 134.8722 123.0093) (end 132.1813 125.7002) (width 0.2) (layer "B.Cu") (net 1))
 (segment (start 103.8 118.8125) (end 92.075 107.0875) (width 0.2) (layer "B.Cu") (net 1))
 (segment (start 115.25 81.1875) (end 115.25 70.645) (width 0.2) (layer "B.Cu") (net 1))
 (segment (start 101.905 70.4237) (end 101.905 71.29) (width 0.2) (layer "B.Cu") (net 1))
 (segment (start 115.25 105) (end 115.25 128.8125) (width 0.2) (layer "B.Cu") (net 1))
 (segment (start 160.95 95) (end 160.95 118.8125) (width 0.2) (layer "B.Cu") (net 1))
 (segment (start 160.95 118.8125) (end 158.8088 120.9537) (width 0.2) (layer "B.Cu") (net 1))
 (segment (start 92.075 107.0875) (end 92.075 102.625) (width 0.2) (layer "B.Cu") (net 1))
 (segment (start 134.3 81.1875) (end 134.3 105) (width 0.2) (layer "B.Cu") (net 1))
 (segment (start 115.25 81.1875) (end 115.25 105) (width 0.2) (layer "B.Cu") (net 1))
 (segment (start 154.7713 120.9537) (end 148.625 127.1) (width 0.2) (layer "B.Cu") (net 1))
 (segment (start 92.075 97.375) (end 92.075 102.625) (width 0.2) (layer "B.Cu") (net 1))
 (segment (start 100.6996 69.2183) (end 101.905 70.4237) (width 0.2) (layer "B.Cu") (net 1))
 (segment (start 101.905 63.67) (end 100.6996 64.8754) (width 0.2) (layer "B.Cu") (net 1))
 (segment (start 134.0442 128.5567) (end 134.3 128.8125) (width 0.2) (layer "B.Cu") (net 1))
 (segment (start 101.905 73.83) (end 101.905 71.29) (width 0.2) (layer "B.Cu") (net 1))
 (segment (start 126.035 116.7) (end 126.035 119.554) (width 0.2) (layer "B.Cu") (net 1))
 (segment (start 115.25 70.645) (end 117.145 68.75) (width 0.2) (layer "B.Cu") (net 1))
 (segment (start 103.6402 92.9204) (end 105.9 95.1802) (width 0.2) (layer "F.Cu") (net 10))
 (segment (start 101.5674 92.9204) (end 103.6402 92.9204) (width 0.2) (layer "F.Cu") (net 10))
 (segment (start 100.7506 85.1444) (end 100.7506 92.1036) (width 0.2) (layer "F.Cu") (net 10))
 (segment (start 101.905 83.99) (end 100.7506 85.1444) (width 0.2) (layer "F.Cu") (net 10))
 (segment (start 105.9 95.1802) (end 105.9 100) (width 0.2) (layer "F.Cu") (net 10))
 (segment (start 100.7506 92.1036) (end 101.5674 92.9204) (width 0.2) (layer "F.Cu") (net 10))
 (segment (start 105.9 82.535) (end 105.9 76.1875) (width 0.2) (layer "B.Cu") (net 7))
 (segment (start 101.905 86.53) (end 105.9 82.535) (width 0.2) (layer "B.Cu") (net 7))
 (segment (start 159.7696 120.5321) (end 163.05 123.8125) (width 0.2) (layer "F.Cu") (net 11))
 (segment (start 155.2783 120.5321) (end 159.7696 120.5321) (width 0.2) (layer "F.Cu") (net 11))
 (segment (start 117.145 91.61) (end 126.3562 91.61) (width 0.2) (layer "F.Cu") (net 11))
 (segment (start 126.3562 91.61) (end 155.2783 120.5321) (width 0.2) (layer "F.Cu") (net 11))
 (segment (start 159.7696 96.7196) (end 163.05 100) (width 0.2) (layer "F.Cu") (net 4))
 (segment (start 117.145 83.99) (end 115.9758 85.1592) (width 0.2) (layer "F.Cu") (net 4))
 (segment (start 148.0636 87.7313) (end 157.0519 96.7196) (width 0.2) (layer "F.Cu") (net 4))
 (segment (start 116.6665 87.7313) (end 148.0636 87.7313) (width 0.2) (layer "F.Cu") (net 4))
 (segment (start 115.9758 87.0406) (end 116.6665 87.7313) (width 0.2) (layer "F.Cu") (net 4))
 (segment (start 157.0519 96.7196) (end 159.7696 96.7196) (width 0.2) (layer "F.Cu") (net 4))
 (segment (start 115.9758 85.1592) (end 115.9758 87.0406) (width 0.2) (layer "F.Cu") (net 4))
 (segment (start 160.7948 73.9323) (end 163.05 76.1875) (width 0.2) (layer "F.Cu") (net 12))
 (segment (start 117.145 81.45) (end 124.6627 73.9323) (width 0.2) (layer "F.Cu") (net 12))
 (segment (start 124.6627 73.9323) (end 160.7948 73.9323) (width 0.2) (layer "F.Cu") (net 12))
 (segment (start 101.905 89.07) (end 109.525 89.07) (width 0.2) (layer "F.Cu") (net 5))
 (via (at 109.525 89.07) (size 0.6) (drill 0.3) (layers "F.Cu" "B.Cu") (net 5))
 (segment (start 113.15 123.8125) (end 109.525 120.1875) (width 0.2) (layer "B.Cu") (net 5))
 (segment (start 109.525 120.1875) (end 109.525 89.07) (width 0.2) (layer "B.Cu") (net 5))
 (segment (start 104.76 91.61) (end 113.15 100) (width 0.2) (layer "F.Cu") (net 3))
 (segment (start 101.905 91.61) (end 104.76 91.61) (width 0.2) (layer "F.Cu") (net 3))
 (segment (start 113.15 83.2723) (end 113.15 76.1875) (width 0.2) (layer "B.Cu") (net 6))
 (segment (start 102.2723 94.15) (end 113.15 83.2723) (width 0.2) (layer "B.Cu") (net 6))
 (segment (start 101.905 94.15) (end 102.2723 94.15) (width 0.2) (layer "B.Cu") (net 6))
 (segment (start 117.145 94.722) (end 127.305 104.882) (width 0.2) (layer "B.Cu") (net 2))
 (segment (start 117.145 94.15) (end 117.145 94.722) (width 0.2) (layer "B.Cu") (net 2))
 (segment (start 127.305 118.9175) (end 132.2 123.8125) (width 0.2) (layer "B.Cu") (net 2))
 (segment (start 127.305 104.882) (end 127.305 118.9175) (width 0.2) (layer "B.Cu") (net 2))
 (segment (start 117.145 89.07) (end 115.9509 90.2641) (width 0.2) (layer "F.Cu") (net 13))
 (segment (start 115.9509 92.0504) (end 116.7862 92.8857) (width 0.2) (layer "F.Cu") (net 13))
 (segment (start 115.9509 90.2641) (end 115.9509 92.0504) (width 0.2) (layer "F.Cu") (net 13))
 (segment (start 125.0857 92.8857) (end 132.2 100) (width 0.2) (layer "F.Cu") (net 13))
 (segment (start 116.7862 92.8857) (end 125.0857 92.8857) (width 0.2) (layer "F.Cu") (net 13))
 (segment (start 127.4875 76.1875) (end 132.2 76.1875) (width 0.2) (layer "F.Cu") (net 8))
 (segment (start 117.145 86.53) (end 127.4875 76.1875) (width 0.2) (layer "F.Cu") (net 8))
 (segment (start 114.7996 79.5379) (end 114.7996 68.5554) (width 0.2) (layer "B.Cu") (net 14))
 (segment (start 108.775 130.0511) (end 114.4739 124.3522) (width 0.2) (layer "B.Cu") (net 14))
 (segment (start 114.7996 68.5554) (end 117.145 66.21) (width 0.2) (layer "B.Cu") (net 14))
 (segment (start 114.4739 122.1705) (end 113.8759 121.5725) (width 0.2) (layer "B.Cu") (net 14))
 (segment (start 108.775 133.765) (end 108.775 130.0511) (width 0.2) (layer "B.Cu") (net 14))
 (segment (start 114.4739 124.3522) (end 114.4739 122.1705) (width 0.2) (layer "B.Cu") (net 14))
 (segment (start 113.8759 121.5725) (end 113.8759 103.0903) (width 0.2) (layer "B.Cu") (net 14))
 (segment (start 114.4714 102.4948) (end 114.4714 99.2214) (width 0.2) (layer "B.Cu") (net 14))
 (segment (start 117.145 63.67) (end 117.145 66.21) (width 0.2) (layer "B.Cu") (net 14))
 (segment (start 113.8759 103.0903) (end 114.4714 102.4948) (width 0.2) (layer "B.Cu") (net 14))
 (segment (start 113.9251 98.6751) (end 113.9251 80.4124) (width 0.2) (layer "B.Cu") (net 14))
 (segment (start 114.4714 99.2214) (end 113.9251 98.6751) (width 0.2) (layer "B.Cu") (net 14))
 (segment (start 113.9251 80.4124) (end 114.7996 79.5379) (width 0.2) (layer "B.Cu") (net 14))
 (segment (start 117.145 71.29) (end 115.7635 72.6715) (width 0.2) (layer "F.Cu") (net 16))
 (segment (start 115.7635 72.6715) (end 93.775 72.6715) (width 0.2) (layer "F.Cu") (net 16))
 (via (at 93.775 72.6715) (size 0.6) (drill 0.3) (layers "F.Cu" "B.Cu") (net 16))
 (segment (start 93.775 97.375) (end 93.775 72.6715) (width 0.2) (layer "B.Cu") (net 16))
 (segment (start 93.775 97.375) (end 93.775 102.625) (width 0.2) (layer "B.Cu") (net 16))
 (segment (start 128.575 116.7) (end 128.575 82.4804) (width 0.2) (layer "B.Cu") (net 17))
 (segment (start 128.575 82.4804) (end 119.9246 73.83) (width 0.2) (layer "B.Cu") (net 17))
 (segment (start 119.9246 73.83) (end 117.145 73.83) (width 0.2) (layer "B.Cu") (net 17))
 (segment (start 117.27 109.3233) (end 117.27 102.2586) (width 0.2) (layer "F.Cu") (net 23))
 (segment (start 117.27 102.2586) (end 114.5876 99.5762) (width 0.2) (layer "F.Cu") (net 23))
 (segment (start 114.5876 99.5762) (end 114.5876 98.3826) (width 0.2) (layer "F.Cu") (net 23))
 (segment (start 114.5876 98.3826) (end 105.8882 89.6832) (width 0.2) (layer "F.Cu") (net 23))
 (segment (start 123.495 116.7) (end 123.495 115.5483) (width 0.2) (layer "F.Cu") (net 23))
 (segment (start 123.495 115.5483) (end 117.27 109.3233) (width 0.2) (layer "F.Cu") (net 23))
 (via (at 105.8882 89.6832) (size 0.6) (drill 0.3) (layers "F.Cu" "B.Cu") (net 23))
 (segment (start 105.8882 89.6832) (end 107.2379 88.3335) (width 0.2) (layer "B.Cu") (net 23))
 (segment (start 107.2379 71.5429) (end 101.905 66.21) (width 0.2) (layer "B.Cu") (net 23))
 (segment (start 107.2379 88.3335) (end 107.2379 71.5429) (width 0.2) (layer "B.Cu") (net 23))
 (segment (start 114.9877 91.9927) (end 114.9877 93.7099) (width 0.2) (layer "F.Cu") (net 20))
 (segment (start 118.8122 97.5344) (end 119.815 97.5344) (width 0.2) (layer "F.Cu") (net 20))
 (segment (start 114.9877 93.7099) (end 118.8122 97.5344) (width 0.2) (layer "F.Cu") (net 20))
 (segment (start 101.905 78.91) (end 114.9877 91.9927) (width 0.2) (layer "F.Cu") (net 20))
 (segment (start 131.115 108.8344) (end 131.115 116.7) (width 0.2) (layer "F.Cu") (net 20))
 (segment (start 119.815 97.5344) (end 131.115 108.8344) (width 0.2) (layer "F.Cu") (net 20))
 (segment (start 140.3658 132.4575) (end 107.275 132.4575) (width 0.2) (layer "F.Cu") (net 15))
 (segment (start 146.625 127.1) (end 145.7233 127.1) (width 0.2) (layer "F.Cu") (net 15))
 (segment (start 145.7233 127.1) (end 140.3658 132.4575) (width 0.2) (layer "F.Cu") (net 15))
 (via (at 107.275 132.4575) (size 0.6) (drill 0.3) (layers "F.Cu" "B.Cu") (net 15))
 (segment (start 107.275 133.765) (end 107.275 132.4575) (width 0.2) (layer "B.Cu") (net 15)))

